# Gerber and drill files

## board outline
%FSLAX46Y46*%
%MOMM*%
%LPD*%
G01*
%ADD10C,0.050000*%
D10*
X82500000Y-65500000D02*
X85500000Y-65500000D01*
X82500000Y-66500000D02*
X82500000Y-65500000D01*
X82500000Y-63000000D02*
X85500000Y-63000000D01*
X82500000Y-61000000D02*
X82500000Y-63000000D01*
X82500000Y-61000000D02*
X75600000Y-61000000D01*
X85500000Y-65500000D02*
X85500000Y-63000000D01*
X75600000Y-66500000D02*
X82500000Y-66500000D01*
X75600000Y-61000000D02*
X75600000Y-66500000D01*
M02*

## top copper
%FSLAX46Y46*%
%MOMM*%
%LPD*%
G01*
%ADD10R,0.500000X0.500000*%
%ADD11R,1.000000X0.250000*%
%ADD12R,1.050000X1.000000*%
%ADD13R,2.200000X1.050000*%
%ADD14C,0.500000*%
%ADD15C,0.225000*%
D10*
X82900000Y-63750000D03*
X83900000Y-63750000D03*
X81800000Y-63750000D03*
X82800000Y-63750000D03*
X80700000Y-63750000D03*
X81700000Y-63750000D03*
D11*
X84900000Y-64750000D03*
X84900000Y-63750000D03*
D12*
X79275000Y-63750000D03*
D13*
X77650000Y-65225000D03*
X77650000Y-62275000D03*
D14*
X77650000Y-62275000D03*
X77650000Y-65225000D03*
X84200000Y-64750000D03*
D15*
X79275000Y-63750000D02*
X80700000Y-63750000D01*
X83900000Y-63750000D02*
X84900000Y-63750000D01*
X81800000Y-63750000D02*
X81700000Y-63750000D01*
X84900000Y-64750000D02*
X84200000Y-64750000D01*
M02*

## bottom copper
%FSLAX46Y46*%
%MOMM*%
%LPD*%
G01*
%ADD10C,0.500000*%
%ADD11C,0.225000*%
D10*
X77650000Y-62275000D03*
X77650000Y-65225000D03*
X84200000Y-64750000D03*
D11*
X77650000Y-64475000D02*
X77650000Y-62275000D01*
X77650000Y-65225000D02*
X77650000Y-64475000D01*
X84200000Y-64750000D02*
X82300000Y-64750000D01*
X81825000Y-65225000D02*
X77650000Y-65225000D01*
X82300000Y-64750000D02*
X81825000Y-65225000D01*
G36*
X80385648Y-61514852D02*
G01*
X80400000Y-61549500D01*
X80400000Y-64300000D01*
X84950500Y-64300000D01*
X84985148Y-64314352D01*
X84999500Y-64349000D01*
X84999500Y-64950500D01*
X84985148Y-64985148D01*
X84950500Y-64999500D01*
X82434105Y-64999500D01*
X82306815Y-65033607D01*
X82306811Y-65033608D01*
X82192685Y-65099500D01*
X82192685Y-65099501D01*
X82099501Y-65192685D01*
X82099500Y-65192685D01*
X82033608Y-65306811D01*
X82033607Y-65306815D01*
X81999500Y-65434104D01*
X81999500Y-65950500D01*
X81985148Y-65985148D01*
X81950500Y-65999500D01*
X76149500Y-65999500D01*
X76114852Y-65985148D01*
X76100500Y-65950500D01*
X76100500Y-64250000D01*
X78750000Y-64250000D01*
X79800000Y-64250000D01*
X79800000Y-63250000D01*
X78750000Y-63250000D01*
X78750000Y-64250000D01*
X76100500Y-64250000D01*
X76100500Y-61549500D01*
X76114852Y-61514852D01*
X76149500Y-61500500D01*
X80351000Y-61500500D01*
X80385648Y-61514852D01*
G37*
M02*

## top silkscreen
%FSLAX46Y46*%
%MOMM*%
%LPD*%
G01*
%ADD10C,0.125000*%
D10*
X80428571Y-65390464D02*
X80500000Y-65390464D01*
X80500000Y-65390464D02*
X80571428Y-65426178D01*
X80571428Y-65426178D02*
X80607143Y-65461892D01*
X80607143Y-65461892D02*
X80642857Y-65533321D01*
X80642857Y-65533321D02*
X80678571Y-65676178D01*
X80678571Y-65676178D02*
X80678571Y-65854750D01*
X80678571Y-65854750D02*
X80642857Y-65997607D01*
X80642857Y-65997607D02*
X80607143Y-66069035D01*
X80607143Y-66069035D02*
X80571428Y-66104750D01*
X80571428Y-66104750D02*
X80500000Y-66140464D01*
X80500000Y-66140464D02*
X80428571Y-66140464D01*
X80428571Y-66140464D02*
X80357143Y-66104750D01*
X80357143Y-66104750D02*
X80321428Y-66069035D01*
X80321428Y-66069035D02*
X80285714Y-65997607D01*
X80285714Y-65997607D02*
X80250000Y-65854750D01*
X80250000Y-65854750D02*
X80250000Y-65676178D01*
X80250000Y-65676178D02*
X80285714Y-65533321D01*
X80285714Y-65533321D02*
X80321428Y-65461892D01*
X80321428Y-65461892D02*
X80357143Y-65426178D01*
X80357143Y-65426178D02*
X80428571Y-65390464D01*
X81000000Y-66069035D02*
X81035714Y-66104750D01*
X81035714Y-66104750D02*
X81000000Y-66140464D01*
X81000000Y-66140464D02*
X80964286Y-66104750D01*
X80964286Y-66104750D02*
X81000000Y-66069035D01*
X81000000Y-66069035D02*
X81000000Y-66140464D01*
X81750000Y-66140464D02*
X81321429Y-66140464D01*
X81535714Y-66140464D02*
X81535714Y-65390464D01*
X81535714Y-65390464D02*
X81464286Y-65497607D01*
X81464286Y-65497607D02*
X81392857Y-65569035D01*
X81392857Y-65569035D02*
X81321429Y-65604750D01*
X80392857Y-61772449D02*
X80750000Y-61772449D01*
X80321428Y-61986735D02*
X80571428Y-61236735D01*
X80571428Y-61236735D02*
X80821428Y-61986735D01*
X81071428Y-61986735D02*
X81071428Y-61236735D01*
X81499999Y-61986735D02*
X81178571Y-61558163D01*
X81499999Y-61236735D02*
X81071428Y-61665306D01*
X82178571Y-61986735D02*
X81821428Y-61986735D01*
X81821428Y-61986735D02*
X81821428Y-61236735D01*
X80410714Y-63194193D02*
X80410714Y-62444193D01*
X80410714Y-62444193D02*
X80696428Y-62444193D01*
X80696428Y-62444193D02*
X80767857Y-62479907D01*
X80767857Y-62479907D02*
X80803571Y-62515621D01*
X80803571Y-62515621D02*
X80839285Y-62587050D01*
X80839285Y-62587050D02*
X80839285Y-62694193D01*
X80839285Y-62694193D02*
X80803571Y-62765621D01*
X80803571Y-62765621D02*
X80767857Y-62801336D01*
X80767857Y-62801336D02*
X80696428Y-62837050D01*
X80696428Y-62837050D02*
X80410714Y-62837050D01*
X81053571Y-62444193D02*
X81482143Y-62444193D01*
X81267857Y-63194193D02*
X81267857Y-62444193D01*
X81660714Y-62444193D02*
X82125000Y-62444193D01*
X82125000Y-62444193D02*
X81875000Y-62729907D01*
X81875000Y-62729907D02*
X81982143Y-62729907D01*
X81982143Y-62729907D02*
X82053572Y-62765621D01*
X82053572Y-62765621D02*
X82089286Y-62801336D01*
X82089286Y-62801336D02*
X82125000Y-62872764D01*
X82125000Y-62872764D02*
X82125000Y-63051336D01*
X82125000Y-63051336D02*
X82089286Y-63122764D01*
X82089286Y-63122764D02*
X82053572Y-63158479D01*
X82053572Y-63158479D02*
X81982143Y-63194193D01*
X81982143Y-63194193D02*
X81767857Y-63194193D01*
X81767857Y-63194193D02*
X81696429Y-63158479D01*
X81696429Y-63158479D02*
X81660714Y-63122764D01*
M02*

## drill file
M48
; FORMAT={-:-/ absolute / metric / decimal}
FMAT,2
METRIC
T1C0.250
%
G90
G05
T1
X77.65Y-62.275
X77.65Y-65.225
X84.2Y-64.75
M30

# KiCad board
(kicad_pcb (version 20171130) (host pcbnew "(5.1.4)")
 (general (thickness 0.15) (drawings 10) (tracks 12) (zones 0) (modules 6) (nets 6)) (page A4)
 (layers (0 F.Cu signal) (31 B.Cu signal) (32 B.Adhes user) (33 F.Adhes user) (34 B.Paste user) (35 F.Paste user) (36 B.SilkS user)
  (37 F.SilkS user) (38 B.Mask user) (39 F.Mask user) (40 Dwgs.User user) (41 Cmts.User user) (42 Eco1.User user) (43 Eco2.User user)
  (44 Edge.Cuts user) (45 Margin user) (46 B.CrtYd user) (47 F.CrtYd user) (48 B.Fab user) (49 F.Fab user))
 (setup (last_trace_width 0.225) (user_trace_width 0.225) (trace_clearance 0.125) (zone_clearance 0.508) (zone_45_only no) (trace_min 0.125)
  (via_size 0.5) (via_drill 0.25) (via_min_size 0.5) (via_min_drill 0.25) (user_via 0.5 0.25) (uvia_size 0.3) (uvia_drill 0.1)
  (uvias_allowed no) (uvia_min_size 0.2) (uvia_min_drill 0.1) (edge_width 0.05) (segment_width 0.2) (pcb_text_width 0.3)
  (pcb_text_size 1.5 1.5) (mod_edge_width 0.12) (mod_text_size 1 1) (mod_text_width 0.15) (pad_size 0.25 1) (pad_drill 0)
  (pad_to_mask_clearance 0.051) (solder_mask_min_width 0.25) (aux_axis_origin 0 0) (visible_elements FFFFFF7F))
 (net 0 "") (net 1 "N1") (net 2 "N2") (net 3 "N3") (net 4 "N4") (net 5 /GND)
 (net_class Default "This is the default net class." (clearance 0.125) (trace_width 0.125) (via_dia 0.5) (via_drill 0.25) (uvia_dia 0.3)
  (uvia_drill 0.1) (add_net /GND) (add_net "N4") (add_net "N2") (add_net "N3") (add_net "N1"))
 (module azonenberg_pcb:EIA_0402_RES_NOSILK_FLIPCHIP (layer F.Cu) (at 83.4 63.75 180) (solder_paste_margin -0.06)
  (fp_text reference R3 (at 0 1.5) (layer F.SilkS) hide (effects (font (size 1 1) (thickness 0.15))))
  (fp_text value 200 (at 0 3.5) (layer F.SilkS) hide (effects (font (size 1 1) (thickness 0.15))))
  (pad 2 smd rect (at 0.5 0 180) (size 0.5 0.5) (layers F.Cu F.Paste F.Mask) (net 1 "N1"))
  (pad 1 smd rect (at -0.5 0 180) (size 0.5 0.5) (layers F.Cu F.Paste F.Mask) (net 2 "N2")))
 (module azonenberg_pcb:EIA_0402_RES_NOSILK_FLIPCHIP (layer F.Cu) (at 82.3 63.75 180) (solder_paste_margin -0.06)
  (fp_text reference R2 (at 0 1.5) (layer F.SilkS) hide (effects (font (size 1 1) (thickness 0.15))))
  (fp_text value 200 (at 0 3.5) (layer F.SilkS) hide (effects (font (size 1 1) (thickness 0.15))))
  (pad 2 smd rect (at 0.5 0 180) (size 0.5 0.5) (layers F.Cu F.Paste F.Mask) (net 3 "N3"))
  (pad 1 smd rect (at -0.5 0 180) (size 0.5 0.5) (layers F.Cu F.Paste F.Mask) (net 1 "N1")))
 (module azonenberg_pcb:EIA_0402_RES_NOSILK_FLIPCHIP (layer F.Cu) (at 81.2 63.75 180) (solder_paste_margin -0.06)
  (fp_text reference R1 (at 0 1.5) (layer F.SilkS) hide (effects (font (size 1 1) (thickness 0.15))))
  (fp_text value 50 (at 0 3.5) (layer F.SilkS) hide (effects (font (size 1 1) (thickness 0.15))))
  (pad 2 smd rect (at 0.5 0 180) (size 0.5 0.5) (layers F.Cu F.Paste F.Mask) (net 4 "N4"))
  (pad 1 smd rect (at -0.5 0 180) (size 0.5 0.5) (layers F.Cu F.Paste F.Mask) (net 3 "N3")))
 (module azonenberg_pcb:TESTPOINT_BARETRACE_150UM (layer F.Cu) (at 84.9 64.75 90) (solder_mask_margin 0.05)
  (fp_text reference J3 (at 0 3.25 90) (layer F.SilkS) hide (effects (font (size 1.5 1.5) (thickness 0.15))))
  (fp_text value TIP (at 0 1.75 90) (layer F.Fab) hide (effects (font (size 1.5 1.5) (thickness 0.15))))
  (pad 1 smd rect (at 0 0 90) (size 0.25 1) (layers F.Cu F.Mask) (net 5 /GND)))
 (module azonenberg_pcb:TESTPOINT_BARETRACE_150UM (layer F.Cu) (at 84.9 63.75 90) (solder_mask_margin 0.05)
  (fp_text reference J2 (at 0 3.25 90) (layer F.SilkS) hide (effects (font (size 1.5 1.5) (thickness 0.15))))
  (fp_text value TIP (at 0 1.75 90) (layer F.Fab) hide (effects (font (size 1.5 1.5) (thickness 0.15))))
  (pad 1 smd rect (at 0 0 90) (size 0.25 1) (layers F.Cu F.Mask) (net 2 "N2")))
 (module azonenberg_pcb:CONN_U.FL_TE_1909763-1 (layer F.Cu) (at 77.75 63.75 90)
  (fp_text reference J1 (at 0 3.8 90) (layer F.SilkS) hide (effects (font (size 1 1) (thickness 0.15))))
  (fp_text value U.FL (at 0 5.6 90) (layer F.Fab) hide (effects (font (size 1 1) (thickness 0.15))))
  (pad 1 smd rect (at 0 1.525 90) (size 1 1.05) (layers F.Cu F.Paste F.Mask) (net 4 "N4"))
  (pad 2 smd rect (at -1.475 -0.1 90) (size 1.05 2.2) (layers F.Cu F.Paste F.Mask) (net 5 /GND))
  (pad 2 smd rect (at 1.475 -0.1 90) (size 1.05 2.2) (layers F.Cu F.Paste F.Mask) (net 5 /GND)))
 (gr_line (start 82.5 65.5) (end 85.5 65.5) (layer Edge.Cuts) (width 0.05))
 (gr_line (start 82.5 66.5) (end 82.5 65.5) (layer Edge.Cuts) (width 0.05))
 (gr_line (start 82.5 63) (end 85.5 63) (layer Edge.Cuts) (width 0.05))
 (gr_line (start 82.5 61) (end 82.5 63) (layer Edge.Cuts) (width 0.05))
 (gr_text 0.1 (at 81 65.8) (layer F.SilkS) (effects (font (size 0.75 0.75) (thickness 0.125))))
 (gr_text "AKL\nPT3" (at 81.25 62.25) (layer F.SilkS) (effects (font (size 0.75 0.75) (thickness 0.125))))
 (gr_line (start 82.5 61) (end 75.6 61) (layer Edge.Cuts) (width 0.05))
 (gr_line (start 85.5 65.5) (end 85.5 63) (layer Edge.Cuts) (width 0.05))
 (gr_line (start 75.6 66.5) (end 82.5 66.5) (layer Edge.Cuts) (width 0.05))
 (gr_line (start 75.6 61) (end 75.6 66.5) (layer Edge.Cuts) (width 0.05))
 (segment (start 79.275 63.75) (end 80.7 63.75) (width 0.225) (layer F.Cu) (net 4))
 (segment (start 83.9 63.75) (end 84.9 63.75) (width 0.225) (layer F.Cu) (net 2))
 (segment (start 81.8 63.75) (end 81.7 63.75) (width 0.225) (layer F.Cu) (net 3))
 (via (at 77.65 62.275) (size 0.5) (drill 0.25) (layers F.Cu B.Cu) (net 5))
 (via (at 77.65 65.225) (size 0.5) (drill 0.25) (layers F.Cu B.Cu) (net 5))
 (segment (start 77.65 64.475) (end 77.65 62.275) (width 0.225) (layer B.Cu) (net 5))
 (segment (start 77.65 65.225) (end 77.65 64.475) (width 0.225) (layer B.Cu) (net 5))
 (via (at 84.2 64.75) (size 0.5) (drill 0.25) (layers F.Cu B.Cu) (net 5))
 (segment (start 84.9 64.75) (end 84.2 64.75) (width 0.225) (layer F.Cu) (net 5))
 (segment (start 84.2 64.75) (end 82.3 64.75) (width 0.225) (layer B.Cu) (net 5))
 (segment (start 81.825 65.225) (end 77.65 65.225) (width 0.225) (layer B.Cu) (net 5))
 (segment (start 82.3 64.75) (end 81.825 65.225) (width 0.225) (layer B.Cu) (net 5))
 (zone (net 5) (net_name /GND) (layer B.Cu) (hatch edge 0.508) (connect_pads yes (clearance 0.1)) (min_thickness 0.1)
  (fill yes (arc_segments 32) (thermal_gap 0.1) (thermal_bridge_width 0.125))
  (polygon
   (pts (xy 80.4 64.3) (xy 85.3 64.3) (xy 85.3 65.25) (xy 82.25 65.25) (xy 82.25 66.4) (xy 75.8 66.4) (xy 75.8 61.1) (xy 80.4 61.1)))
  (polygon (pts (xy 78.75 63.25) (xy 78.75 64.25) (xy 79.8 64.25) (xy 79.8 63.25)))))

